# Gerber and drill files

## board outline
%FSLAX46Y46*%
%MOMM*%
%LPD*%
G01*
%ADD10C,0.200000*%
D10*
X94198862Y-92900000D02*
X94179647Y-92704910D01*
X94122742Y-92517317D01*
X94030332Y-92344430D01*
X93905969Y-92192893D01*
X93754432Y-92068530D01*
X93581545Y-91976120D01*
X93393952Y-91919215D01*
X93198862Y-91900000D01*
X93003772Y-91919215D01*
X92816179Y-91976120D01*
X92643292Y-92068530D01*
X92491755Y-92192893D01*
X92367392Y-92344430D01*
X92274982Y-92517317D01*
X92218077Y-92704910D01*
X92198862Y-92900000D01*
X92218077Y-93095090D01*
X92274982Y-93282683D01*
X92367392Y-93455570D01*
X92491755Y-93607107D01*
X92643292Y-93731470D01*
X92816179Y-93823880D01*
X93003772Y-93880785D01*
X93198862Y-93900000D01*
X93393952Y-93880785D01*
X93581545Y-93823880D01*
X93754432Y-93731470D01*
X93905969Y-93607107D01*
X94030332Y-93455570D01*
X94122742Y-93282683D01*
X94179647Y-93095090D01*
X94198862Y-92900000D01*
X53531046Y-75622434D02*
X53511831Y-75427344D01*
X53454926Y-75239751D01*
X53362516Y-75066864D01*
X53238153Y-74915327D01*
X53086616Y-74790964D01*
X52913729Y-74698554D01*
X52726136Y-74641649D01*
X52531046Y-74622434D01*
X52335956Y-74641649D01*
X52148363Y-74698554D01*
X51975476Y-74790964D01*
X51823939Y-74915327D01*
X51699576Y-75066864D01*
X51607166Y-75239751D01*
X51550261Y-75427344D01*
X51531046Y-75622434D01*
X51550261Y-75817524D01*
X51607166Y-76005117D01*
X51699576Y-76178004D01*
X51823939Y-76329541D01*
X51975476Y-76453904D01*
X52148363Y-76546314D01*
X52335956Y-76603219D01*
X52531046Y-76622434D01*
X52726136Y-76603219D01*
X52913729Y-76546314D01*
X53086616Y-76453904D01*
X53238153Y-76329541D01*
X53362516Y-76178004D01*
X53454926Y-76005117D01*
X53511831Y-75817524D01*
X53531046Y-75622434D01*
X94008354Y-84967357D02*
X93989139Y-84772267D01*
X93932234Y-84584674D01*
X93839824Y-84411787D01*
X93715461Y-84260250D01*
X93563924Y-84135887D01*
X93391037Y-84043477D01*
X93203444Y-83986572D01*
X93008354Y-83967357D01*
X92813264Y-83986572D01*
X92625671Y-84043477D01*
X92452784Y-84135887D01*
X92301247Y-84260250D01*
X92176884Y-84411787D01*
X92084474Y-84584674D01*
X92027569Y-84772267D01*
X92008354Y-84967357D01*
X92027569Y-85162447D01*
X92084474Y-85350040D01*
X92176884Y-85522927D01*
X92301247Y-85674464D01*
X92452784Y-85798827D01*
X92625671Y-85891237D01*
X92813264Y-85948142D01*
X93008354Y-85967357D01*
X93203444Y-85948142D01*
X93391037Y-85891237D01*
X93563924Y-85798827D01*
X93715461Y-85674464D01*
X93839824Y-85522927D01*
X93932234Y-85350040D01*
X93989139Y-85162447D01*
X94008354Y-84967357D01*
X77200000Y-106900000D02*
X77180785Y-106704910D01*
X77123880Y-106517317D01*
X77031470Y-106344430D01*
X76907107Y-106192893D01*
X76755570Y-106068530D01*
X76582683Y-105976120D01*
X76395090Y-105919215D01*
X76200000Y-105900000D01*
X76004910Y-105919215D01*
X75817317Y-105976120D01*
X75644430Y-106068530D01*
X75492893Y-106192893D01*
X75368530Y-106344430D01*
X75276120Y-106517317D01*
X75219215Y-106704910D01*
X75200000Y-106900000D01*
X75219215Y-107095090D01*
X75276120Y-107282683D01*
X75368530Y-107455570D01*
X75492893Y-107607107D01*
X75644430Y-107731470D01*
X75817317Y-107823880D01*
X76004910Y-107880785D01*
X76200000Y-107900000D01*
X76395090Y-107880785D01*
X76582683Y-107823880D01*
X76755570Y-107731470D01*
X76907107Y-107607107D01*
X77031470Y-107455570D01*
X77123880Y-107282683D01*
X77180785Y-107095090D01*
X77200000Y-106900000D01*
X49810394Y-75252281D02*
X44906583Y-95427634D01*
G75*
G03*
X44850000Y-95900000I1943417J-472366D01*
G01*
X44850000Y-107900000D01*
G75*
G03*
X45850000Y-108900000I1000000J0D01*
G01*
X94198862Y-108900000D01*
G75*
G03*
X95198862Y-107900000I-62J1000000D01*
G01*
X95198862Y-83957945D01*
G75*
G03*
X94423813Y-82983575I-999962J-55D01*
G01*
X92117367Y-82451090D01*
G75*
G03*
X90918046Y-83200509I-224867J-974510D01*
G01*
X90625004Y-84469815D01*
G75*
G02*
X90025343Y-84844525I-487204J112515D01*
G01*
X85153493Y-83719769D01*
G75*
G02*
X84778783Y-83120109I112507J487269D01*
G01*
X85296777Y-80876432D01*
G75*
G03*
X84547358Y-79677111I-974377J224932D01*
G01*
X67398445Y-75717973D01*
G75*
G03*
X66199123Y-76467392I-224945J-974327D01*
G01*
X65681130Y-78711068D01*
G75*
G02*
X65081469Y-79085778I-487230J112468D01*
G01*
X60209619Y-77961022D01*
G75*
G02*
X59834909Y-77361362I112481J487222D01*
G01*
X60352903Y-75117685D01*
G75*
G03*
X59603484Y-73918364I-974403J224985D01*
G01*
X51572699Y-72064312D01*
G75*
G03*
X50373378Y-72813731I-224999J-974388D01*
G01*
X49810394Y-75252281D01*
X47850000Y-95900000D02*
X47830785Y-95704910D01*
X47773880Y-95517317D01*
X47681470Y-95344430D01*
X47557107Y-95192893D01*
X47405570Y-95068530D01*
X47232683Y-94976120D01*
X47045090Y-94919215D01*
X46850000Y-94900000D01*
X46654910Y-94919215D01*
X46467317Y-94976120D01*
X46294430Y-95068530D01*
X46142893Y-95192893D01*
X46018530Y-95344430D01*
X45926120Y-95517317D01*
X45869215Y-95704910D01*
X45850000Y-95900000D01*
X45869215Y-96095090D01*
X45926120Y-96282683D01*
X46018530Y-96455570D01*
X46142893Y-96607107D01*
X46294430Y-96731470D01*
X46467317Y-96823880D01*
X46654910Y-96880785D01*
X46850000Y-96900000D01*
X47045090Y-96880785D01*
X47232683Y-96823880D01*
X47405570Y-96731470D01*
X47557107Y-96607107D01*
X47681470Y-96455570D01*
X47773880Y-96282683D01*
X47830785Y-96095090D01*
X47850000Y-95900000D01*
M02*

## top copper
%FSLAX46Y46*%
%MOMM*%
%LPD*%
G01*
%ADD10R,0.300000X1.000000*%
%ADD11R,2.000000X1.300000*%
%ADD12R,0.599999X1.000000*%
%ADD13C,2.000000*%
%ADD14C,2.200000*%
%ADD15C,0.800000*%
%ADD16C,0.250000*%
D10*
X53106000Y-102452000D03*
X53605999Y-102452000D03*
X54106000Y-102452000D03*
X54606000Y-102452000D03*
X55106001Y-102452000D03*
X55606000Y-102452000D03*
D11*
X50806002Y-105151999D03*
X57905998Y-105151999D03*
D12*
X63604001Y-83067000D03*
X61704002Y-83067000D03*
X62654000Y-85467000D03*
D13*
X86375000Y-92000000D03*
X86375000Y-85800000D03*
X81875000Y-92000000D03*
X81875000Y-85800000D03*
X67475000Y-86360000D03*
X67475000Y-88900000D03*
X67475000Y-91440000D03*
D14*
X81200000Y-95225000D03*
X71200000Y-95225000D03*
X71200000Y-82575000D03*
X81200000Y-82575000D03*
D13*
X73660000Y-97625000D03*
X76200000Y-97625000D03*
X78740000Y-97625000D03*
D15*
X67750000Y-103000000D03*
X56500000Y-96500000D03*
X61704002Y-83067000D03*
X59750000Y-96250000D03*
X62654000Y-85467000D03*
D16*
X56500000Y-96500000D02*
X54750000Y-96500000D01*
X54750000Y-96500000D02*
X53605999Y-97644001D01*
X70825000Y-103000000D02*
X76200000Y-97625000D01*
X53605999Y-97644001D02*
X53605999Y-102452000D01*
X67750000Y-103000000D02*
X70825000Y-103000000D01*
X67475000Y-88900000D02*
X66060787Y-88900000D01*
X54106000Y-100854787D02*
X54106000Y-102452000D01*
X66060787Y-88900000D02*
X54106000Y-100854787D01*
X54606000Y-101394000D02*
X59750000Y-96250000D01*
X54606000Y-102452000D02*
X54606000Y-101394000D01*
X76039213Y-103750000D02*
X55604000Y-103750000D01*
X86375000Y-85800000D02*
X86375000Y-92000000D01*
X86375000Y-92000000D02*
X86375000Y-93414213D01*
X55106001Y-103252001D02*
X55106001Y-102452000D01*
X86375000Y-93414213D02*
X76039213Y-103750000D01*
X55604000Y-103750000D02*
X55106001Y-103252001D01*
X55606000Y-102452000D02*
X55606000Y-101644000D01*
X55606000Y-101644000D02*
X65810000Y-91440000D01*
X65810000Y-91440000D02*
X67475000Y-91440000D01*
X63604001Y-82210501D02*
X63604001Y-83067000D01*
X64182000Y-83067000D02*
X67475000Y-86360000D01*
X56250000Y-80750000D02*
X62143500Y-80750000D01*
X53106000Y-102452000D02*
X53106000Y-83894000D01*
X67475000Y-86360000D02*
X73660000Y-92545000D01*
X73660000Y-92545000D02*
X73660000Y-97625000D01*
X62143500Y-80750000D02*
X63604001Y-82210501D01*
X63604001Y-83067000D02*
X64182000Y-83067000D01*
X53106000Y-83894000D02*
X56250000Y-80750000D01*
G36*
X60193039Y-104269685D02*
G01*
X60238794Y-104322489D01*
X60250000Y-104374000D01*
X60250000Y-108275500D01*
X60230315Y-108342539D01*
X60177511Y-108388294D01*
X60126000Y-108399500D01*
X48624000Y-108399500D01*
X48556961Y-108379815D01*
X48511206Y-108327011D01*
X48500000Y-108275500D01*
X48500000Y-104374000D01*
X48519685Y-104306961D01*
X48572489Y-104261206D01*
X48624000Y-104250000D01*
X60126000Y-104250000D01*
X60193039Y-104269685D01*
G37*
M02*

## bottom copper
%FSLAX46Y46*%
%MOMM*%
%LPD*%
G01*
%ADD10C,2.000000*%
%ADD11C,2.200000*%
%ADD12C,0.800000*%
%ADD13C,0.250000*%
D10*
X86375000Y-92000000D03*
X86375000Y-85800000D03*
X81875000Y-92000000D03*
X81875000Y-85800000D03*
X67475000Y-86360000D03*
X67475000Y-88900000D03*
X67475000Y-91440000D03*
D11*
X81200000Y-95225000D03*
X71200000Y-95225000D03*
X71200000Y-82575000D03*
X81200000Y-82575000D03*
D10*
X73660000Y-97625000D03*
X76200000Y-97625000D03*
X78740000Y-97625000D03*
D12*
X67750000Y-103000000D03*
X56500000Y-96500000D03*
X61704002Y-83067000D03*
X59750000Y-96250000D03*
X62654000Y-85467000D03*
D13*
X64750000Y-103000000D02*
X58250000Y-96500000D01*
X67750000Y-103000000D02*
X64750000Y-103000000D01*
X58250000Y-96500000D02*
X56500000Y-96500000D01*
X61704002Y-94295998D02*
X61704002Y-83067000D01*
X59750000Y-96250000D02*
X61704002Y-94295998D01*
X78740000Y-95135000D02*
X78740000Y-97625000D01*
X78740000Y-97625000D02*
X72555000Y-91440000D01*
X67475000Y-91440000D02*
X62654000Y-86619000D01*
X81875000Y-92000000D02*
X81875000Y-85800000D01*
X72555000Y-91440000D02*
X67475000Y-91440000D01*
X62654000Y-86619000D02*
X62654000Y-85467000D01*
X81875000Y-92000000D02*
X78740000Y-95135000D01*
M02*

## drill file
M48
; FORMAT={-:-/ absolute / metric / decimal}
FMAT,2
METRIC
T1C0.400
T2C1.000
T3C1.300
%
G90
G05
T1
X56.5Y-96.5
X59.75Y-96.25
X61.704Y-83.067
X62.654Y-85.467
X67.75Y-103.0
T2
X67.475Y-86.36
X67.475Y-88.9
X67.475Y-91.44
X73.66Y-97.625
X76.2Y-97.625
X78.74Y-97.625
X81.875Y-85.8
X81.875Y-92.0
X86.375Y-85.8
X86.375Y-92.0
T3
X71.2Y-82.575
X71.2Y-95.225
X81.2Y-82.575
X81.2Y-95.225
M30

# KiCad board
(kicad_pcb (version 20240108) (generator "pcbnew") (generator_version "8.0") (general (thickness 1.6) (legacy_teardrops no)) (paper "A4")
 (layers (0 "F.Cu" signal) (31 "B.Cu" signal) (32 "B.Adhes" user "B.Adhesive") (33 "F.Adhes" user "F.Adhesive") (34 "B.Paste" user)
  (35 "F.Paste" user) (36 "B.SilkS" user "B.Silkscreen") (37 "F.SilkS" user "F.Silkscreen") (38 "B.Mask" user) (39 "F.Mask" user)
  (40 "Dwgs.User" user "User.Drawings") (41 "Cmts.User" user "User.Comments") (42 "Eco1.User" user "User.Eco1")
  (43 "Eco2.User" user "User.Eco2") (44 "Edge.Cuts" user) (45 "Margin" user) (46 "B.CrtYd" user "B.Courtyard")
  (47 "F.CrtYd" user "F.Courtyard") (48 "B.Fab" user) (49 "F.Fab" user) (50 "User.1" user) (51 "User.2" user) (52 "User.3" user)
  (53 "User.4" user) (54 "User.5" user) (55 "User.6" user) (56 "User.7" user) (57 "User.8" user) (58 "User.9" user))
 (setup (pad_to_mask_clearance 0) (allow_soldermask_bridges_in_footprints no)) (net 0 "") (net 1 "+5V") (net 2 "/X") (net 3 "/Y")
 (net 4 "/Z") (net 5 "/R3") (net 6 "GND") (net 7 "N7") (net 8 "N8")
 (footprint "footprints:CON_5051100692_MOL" (layer "F.Cu") (at 54.356 104.902)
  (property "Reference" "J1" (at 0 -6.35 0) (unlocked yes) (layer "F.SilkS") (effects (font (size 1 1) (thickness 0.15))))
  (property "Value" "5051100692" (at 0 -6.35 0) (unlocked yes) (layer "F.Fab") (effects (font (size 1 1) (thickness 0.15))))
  (pad "1" smd rect (at -1.25 -2.45) (size 0.3 1) (layers "F.Cu" "F.Paste" "F.Mask") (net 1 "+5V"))
  (pad "2" smd rect (at -0.750001 -2.45) (size 0.3 1) (layers "F.Cu" "F.Paste" "F.Mask") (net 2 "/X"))
  (pad "3" smd rect (at -0.25 -2.45) (size 0.3 1) (layers "F.Cu" "F.Paste" "F.Mask") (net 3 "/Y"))
  (pad "4" smd rect (at 0.25 -2.45) (size 0.3 1) (layers "F.Cu" "F.Paste" "F.Mask") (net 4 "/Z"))
  (pad "5" smd rect (at 0.750001 -2.45) (size 0.3 1) (layers "F.Cu" "F.Paste" "F.Mask") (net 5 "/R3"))
  (pad "6" smd rect (at 1.25 -2.45) (size 0.3 1) (layers "F.Cu" "F.Paste" "F.Mask") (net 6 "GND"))
  (pad "P1" smd rect (at -3.549998 0.249999) (size 2 1.3) (layers "F.Cu" "F.Paste" "F.Mask") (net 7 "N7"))
  (pad "P2" smd rect (at 3.549998 0.249999) (size 2 1.3) (layers "F.Cu" "F.Paste" "F.Mask") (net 7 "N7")))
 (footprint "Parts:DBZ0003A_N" (layer "F.Cu") (at 62.654 84.267 -90)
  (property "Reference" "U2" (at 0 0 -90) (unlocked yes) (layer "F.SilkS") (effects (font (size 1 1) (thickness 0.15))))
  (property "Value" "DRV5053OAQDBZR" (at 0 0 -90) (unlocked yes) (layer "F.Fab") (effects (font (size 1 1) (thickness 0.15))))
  (pad "1" smd rect (at -1.2 -0.950001) (size 0.599999 1) (layers "F.Cu" "F.Paste" "F.Mask") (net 1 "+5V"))
  (pad "2" smd rect (at -1.2 0.949998) (size 0.599999 1) (layers "F.Cu" "F.Paste" "F.Mask") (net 4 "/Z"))
  (pad "3" smd rect (at 1.2 0) (size 0.599999 1) (layers "F.Cu" "F.Paste" "F.Mask") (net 6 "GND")))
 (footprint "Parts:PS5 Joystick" (layer "B.Cu") (at 76.2 88.9 180)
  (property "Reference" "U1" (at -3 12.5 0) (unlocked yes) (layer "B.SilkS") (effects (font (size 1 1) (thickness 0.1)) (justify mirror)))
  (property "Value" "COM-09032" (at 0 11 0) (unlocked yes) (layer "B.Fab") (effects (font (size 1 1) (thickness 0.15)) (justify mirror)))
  (pad "B1A" thru_hole circle (at -10.175 -3.1 180) (size 2 2) (drill 1) (layers "*.Cu" "*.Mask") (remove_unused_layers no) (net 5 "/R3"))
  (pad "B1A" thru_hole circle (at -10.175 3.1 180) (size 2 2) (drill 1) (layers "*.Cu" "*.Mask") (remove_unused_layers no) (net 5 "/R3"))
  (pad "B2A" thru_hole circle (at -5.675 -3.1 180) (size 2 2) (drill 1) (layers "*.Cu" "*.Mask") (remove_unused_layers no) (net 6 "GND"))
  (pad "B2A" thru_hole circle (at -5.675 3.1 180) (size 2 2) (drill 1) (layers "*.Cu" "*.Mask") (remove_unused_layers no) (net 6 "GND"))
  (pad "H1" thru_hole circle (at 8.725 2.54 180) (size 2 2) (drill 1) (layers "*.Cu" "*.Mask") (remove_unused_layers no) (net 1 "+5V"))
  (pad "H2" thru_hole circle (at 8.725 0 180) (size 2 2) (drill 1) (layers "*.Cu" "*.Mask") (remove_unused_layers no) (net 3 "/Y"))
  (pad "H3" thru_hole circle (at 8.725 -2.54 180) (size 2 2) (drill 1) (layers "*.Cu" "*.Mask") (remove_unused_layers no) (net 6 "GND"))
  (pad "S1" thru_hole circle (at -5 -6.325 180) (size 2.2 2.2) (drill 1.3) (layers "*.Cu" "*.Mask") (remove_unused_layers no) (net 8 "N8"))
  (pad "S2" thru_hole circle (at 5 -6.325 180) (size 2.2 2.2) (drill 1.3) (layers "*.Cu" "*.Mask") (remove_unused_layers no) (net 8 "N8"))
  (pad "S3" thru_hole circle (at 5 6.325 180) (size 2.2 2.2) (drill 1.3) (layers "*.Cu" "*.Mask") (remove_unused_layers no) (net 8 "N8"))
  (pad "S4" thru_hole circle (at -5 6.325 180) (size 2.2 2.2) (drill 1.3) (layers "*.Cu" "*.Mask") (remove_unused_layers no) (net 8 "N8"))
  (pad "V1" thru_hole circle (at 2.54 -8.725 180) (size 2 2) (drill 1) (layers "*.Cu" "*.Mask") (remove_unused_layers no) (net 1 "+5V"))
  (pad "V2" thru_hole circle (at 0 -8.725 180) (size 2 2) (drill 1) (layers "*.Cu" "*.Mask") (remove_unused_layers no) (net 2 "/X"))
  (pad "V3" thru_hole circle (at -2.54 -8.725 180) (size 2 2) (drill 1) (layers "*.Cu" "*.Mask") (remove_unused_layers no) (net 6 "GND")))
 (gr_poly
  (pts (xy 94.198862 92.9) (xy 94.179647 92.70491) (xy 94.122742 92.517317) (xy 94.030332 92.34443) (xy 93.905969 92.192893)
   (xy 93.754432 92.06853) (xy 93.581545 91.97612) (xy 93.393952 91.919215) (xy 93.198862 91.9) (xy 93.003772 91.919215)
   (xy 92.816179 91.97612) (xy 92.643292 92.06853) (xy 92.491755 92.192893) (xy 92.367392 92.34443) (xy 92.274982 92.517317)
   (xy 92.218077 92.70491) (xy 92.198862 92.9) (xy 92.218077 93.09509) (xy 92.274982 93.282683) (xy 92.367392 93.45557)
   (xy 92.491755 93.607107) (xy 92.643292 93.73147) (xy 92.816179 93.82388) (xy 93.003772 93.880785) (xy 93.198862 93.9)
   (xy 93.393952 93.880785) (xy 93.581545 93.82388) (xy 93.754432 93.73147) (xy 93.905969 93.607107) (xy 94.030332 93.45557)
   (xy 94.122742 93.282683) (xy 94.179647 93.09509) (xy 94.198862 92.9))
  (stroke (width 0.2) (type solid)) (fill none) (layer "Edge.Cuts"))
 (gr_poly
  (pts (xy 53.531046 75.622434) (xy 53.511831 75.427344) (xy 53.454926 75.239751) (xy 53.362516 75.066864) (xy 53.238153 74.915327)
   (xy 53.086616 74.790964) (xy 52.913729 74.698554) (xy 52.726136 74.641649) (xy 52.531046 74.622434) (xy 52.335956 74.641649)
   (xy 52.148363 74.698554) (xy 51.975476 74.790964) (xy 51.823939 74.915327) (xy 51.699576 75.066864) (xy 51.607166 75.239751)
   (xy 51.550261 75.427344) (xy 51.531046 75.622434) (xy 51.550261 75.817524) (xy 51.607166 76.005117) (xy 51.699576 76.178004)
   (xy 51.823939 76.329541) (xy 51.975476 76.453904) (xy 52.148363 76.546314) (xy 52.335956 76.603219) (xy 52.531046 76.622434)
   (xy 52.726136 76.603219) (xy 52.913729 76.546314) (xy 53.086616 76.453904) (xy 53.238153 76.329541) (xy 53.362516 76.178004)
   (xy 53.454926 76.005117) (xy 53.511831 75.817524) (xy 53.531046 75.622434))
  (stroke (width 0.2) (type solid)) (fill none) (layer "Edge.Cuts"))
 (gr_poly
  (pts (xy 94.008354 84.967357) (xy 93.989139 84.772267) (xy 93.932234 84.584674) (xy 93.839824 84.411787) (xy 93.715461 84.26025)
   (xy 93.563924 84.135887) (xy 93.391037 84.043477) (xy 93.203444 83.986572) (xy 93.008354 83.967357) (xy 92.813264 83.986572)
   (xy 92.625671 84.043477) (xy 92.452784 84.135887) (xy 92.301247 84.26025) (xy 92.176884 84.411787) (xy 92.084474 84.584674)
   (xy 92.027569 84.772267) (xy 92.008354 84.967357) (xy 92.027569 85.162447) (xy 92.084474 85.35004) (xy 92.176884 85.522927)
   (xy 92.301247 85.674464) (xy 92.452784 85.798827) (xy 92.625671 85.891237) (xy 92.813264 85.948142) (xy 93.008354 85.967357)
   (xy 93.203444 85.948142) (xy 93.391037 85.891237) (xy 93.563924 85.798827) (xy 93.715461 85.674464) (xy 93.839824 85.522927)
   (xy 93.932234 85.35004) (xy 93.989139 85.162447) (xy 94.008354 84.967357))
  (stroke (width 0.2) (type solid)) (fill none) (layer "Edge.Cuts"))
 (gr_poly
  (pts (xy 77.2 106.9) (xy 77.180785 106.70491) (xy 77.12388 106.517317) (xy 77.03147 106.34443) (xy 76.907107 106.192893)
   (xy 76.75557 106.06853) (xy 76.582683 105.97612) (xy 76.39509 105.919215) (xy 76.2 105.9) (xy 76.00491 105.919215)
   (xy 75.817317 105.97612) (xy 75.64443 106.06853) (xy 75.492893 106.192893) (xy 75.36853 106.34443) (xy 75.27612 106.517317)
   (xy 75.219215 106.70491) (xy 75.2 106.9) (xy 75.219215 107.09509) (xy 75.27612 107.282683) (xy 75.36853 107.45557)
   (xy 75.492893 107.607107) (xy 75.64443 107.73147) (xy 75.817317 107.82388) (xy 76.00491 107.880785) (xy 76.2 107.9)
   (xy 76.39509 107.880785) (xy 76.582683 107.82388) (xy 76.75557 107.73147) (xy 76.907107 107.607107) (xy 77.03147 107.45557)
   (xy 77.12388 107.282683) (xy 77.180785 107.09509) (xy 77.2 106.9))
  (stroke (width 0.2) (type solid)) (fill none) (layer "Edge.Cuts"))
 (gr_poly
  (pts (xy 49.810394 75.252281)
   (arc (start 44.906583 95.427634) (mid 44.864196 95.662129) (end 44.85 95.9))
   (arc (start 44.85 107.9) (mid 45.142893 108.607107) (end 45.85 108.9))
   (arc (start 94.198862 108.9) (mid 94.905966 108.607093) (end 95.198862 107.9))
   (arc (start 95.198862 83.957945) (mid 94.981467 83.335431) (end 94.423813 82.983575))
   (arc (start 92.117367 82.45109) (mid 91.362505 82.577445) (end 90.918046 83.200509))
   (arc (start 90.625004 84.469815) (mid 90.402771 84.781349) (end 90.025343 84.844525))
   (arc (start 85.153493 83.719769) (mid 84.841972 83.497537) (end 84.778783 83.120109))
   (arc (start 85.296777 80.876432) (mid 85.170456 80.121561) (end 84.547358 79.677111))
   (arc (start 67.398445 75.717973) (mid 66.643574 75.844295) (end 66.199123 76.467392))
   (arc (start 65.68113 78.711068) (mid 65.458904 79.022617) (end 65.081469 79.085778))
   (arc (start 60.209619 77.961022) (mid 59.89807 77.738797) (end 59.834909 77.361362))
   (arc (start 60.352903 75.117685) (mid 60.226581 74.362815) (end 59.603484 73.918364))
   (arc (start 51.572699 72.064312) (mid 50.817829 72.190634) (end 50.373378 72.813731)))
  (stroke (width 0.2) (type solid)) (fill none) (layer "Edge.Cuts"))
 (gr_poly
  (pts (xy 47.85 95.9) (xy 47.830785 95.70491) (xy 47.77388 95.517317) (xy 47.68147 95.34443) (xy 47.557107 95.192893)
   (xy 47.40557 95.06853) (xy 47.232683 94.97612) (xy 47.04509 94.919215) (xy 46.85 94.9) (xy 46.65491 94.919215) (xy 46.467317 94.97612)
   (xy 46.29443 95.06853) (xy 46.142893 95.192893) (xy 46.01853 95.34443) (xy 45.92612 95.517317) (xy 45.869215 95.70491) (xy 45.85 95.9)
   (xy 45.869215 96.09509) (xy 45.92612 96.282683) (xy 46.01853 96.45557) (xy 46.142893 96.607107) (xy 46.29443 96.73147)
   (xy 46.467317 96.82388) (xy 46.65491 96.880785) (xy 46.85 96.9) (xy 47.04509 96.880785) (xy 47.232683 96.82388) (xy 47.40557 96.73147)
   (xy 47.557107 96.607107) (xy 47.68147 96.45557) (xy 47.77388 96.282683) (xy 47.830785 96.09509) (xy 47.85 95.9))
  (stroke (width 0.2) (type solid)) (fill none) (layer "Edge.Cuts"))
 (segment (start 56.5 96.5) (end 54.75 96.5) (width 0.25) (layer "F.Cu") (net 2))
 (segment (start 54.75 96.5) (end 53.605999 97.644001) (width 0.25) (layer "F.Cu") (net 2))
 (segment (start 70.825 103) (end 76.2 97.625) (width 0.25) (layer "F.Cu") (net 2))
 (segment (start 53.605999 97.644001) (end 53.605999 102.452) (width 0.25) (layer "F.Cu") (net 2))
 (segment (start 67.75 103) (end 70.825 103) (width 0.25) (layer "F.Cu") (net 2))
 (via (at 67.75 103) (size 0.8) (drill 0.4) (layers "F.Cu" "B.Cu") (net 2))
 (via (at 56.5 96.5) (size 0.8) (drill 0.4) (layers "F.Cu" "B.Cu") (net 2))
 (segment (start 64.75 103) (end 58.25 96.5) (width 0.25) (layer "B.Cu") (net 2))
 (segment (start 67.75 103) (end 64.75 103) (width 0.25) (layer "B.Cu") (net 2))
 (segment (start 58.25 96.5) (end 56.5 96.5) (width 0.25) (layer "B.Cu") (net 2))
 (segment (start 67.475 88.9) (end 66.060787 88.9) (width 0.25) (layer "F.Cu") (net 3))
 (segment (start 54.106 100.854787) (end 54.106 102.452) (width 0.25) (layer "F.Cu") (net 3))
 (segment (start 66.060787 88.9) (end 54.106 100.854787) (width 0.25) (layer "F.Cu") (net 3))
 (segment (start 54.606 101.394) (end 59.75 96.25) (width 0.25) (layer "F.Cu") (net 4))
 (segment (start 54.606 102.452) (end 54.606 101.394) (width 0.25) (layer "F.Cu") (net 4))
 (via (at 61.704002 83.067) (size 0.8) (drill 0.4) (layers "F.Cu" "B.Cu") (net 4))
 (via (at 59.75 96.25) (size 0.8) (drill 0.4) (layers "F.Cu" "B.Cu") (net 4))
 (segment (start 61.704002 94.295998) (end 61.704002 83.067) (width 0.25) (layer "B.Cu") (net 4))
 (segment (start 59.75 96.25) (end 61.704002 94.295998) (width 0.25) (layer "B.Cu") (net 4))
 (segment (start 76.039213 103.75) (end 55.604 103.75) (width 0.25) (layer "F.Cu") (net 5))
 (segment (start 86.375 85.8) (end 86.375 92) (width 0.25) (layer "F.Cu") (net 5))
 (segment (start 86.375 92) (end 86.375 93.414213) (width 0.25) (layer "F.Cu") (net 5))
 (segment (start 55.106001 103.252001) (end 55.106001 102.452) (width 0.25) (layer "F.Cu") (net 5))
 (segment (start 86.375 93.414213) (end 76.039213 103.75) (width 0.25) (layer "F.Cu") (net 5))
 (segment (start 55.604 103.75) (end 55.106001 103.252001) (width 0.25) (layer "F.Cu") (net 5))
 (segment (start 55.606 102.452) (end 55.606 101.644) (width 0.25) (layer "F.Cu") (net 6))
 (segment (start 55.606 101.644) (end 65.81 91.44) (width 0.25) (layer "F.Cu") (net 6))
 (segment (start 65.81 91.44) (end 67.475 91.44) (width 0.25) (layer "F.Cu") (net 6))
 (via (at 62.654 85.467) (size 0.8) (drill 0.4) (layers "F.Cu" "B.Cu") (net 6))
 (segment (start 78.74 95.135) (end 78.74 97.625) (width 0.25) (layer "B.Cu") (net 6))
 (segment (start 78.74 97.625) (end 72.555 91.44) (width 0.25) (layer "B.Cu") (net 6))
 (segment (start 67.475 91.44) (end 62.654 86.619) (width 0.25) (layer "B.Cu") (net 6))
 (segment (start 81.875 92) (end 81.875 85.8) (width 0.25) (layer "B.Cu") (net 6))
 (segment (start 72.555 91.44) (end 67.475 91.44) (width 0.25) (layer "B.Cu") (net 6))
 (segment (start 62.654 86.619) (end 62.654 85.467) (width 0.25) (layer "B.Cu") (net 6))
 (segment (start 81.875 92) (end 78.74 95.135) (width 0.25) (layer "B.Cu") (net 6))
 (segment (start 63.604001 82.210501) (end 63.604001 83.067) (width 0.25) (layer "F.Cu") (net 1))
 (segment (start 64.182 83.067) (end 67.475 86.36) (width 0.25) (layer "F.Cu") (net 1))
 (segment (start 56.25 80.75) (end 62.1435 80.75) (width 0.25) (layer "F.Cu") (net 1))
 (segment (start 53.106 102.452) (end 53.106 83.894) (width 0.25) (layer "F.Cu") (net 1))
 (segment (start 67.475 86.36) (end 73.66 92.545) (width 0.25) (layer "F.Cu") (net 1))
 (segment (start 73.66 92.545) (end 73.66 97.625) (width 0.25) (layer "F.Cu") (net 1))
 (segment (start 62.1435 80.75) (end 63.604001 82.210501) (width 0.25) (layer "F.Cu") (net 1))
 (segment (start 63.604001 83.067) (end 64.182 83.067) (width 0.25) (layer "F.Cu") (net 1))
 (segment (start 53.106 83.894) (end 56.25 80.75) (width 0.25) (layer "F.Cu") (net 1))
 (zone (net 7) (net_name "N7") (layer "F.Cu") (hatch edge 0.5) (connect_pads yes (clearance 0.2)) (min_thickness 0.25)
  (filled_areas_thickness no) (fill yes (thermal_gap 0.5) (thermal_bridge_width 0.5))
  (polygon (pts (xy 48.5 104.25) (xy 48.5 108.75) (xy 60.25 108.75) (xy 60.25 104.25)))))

